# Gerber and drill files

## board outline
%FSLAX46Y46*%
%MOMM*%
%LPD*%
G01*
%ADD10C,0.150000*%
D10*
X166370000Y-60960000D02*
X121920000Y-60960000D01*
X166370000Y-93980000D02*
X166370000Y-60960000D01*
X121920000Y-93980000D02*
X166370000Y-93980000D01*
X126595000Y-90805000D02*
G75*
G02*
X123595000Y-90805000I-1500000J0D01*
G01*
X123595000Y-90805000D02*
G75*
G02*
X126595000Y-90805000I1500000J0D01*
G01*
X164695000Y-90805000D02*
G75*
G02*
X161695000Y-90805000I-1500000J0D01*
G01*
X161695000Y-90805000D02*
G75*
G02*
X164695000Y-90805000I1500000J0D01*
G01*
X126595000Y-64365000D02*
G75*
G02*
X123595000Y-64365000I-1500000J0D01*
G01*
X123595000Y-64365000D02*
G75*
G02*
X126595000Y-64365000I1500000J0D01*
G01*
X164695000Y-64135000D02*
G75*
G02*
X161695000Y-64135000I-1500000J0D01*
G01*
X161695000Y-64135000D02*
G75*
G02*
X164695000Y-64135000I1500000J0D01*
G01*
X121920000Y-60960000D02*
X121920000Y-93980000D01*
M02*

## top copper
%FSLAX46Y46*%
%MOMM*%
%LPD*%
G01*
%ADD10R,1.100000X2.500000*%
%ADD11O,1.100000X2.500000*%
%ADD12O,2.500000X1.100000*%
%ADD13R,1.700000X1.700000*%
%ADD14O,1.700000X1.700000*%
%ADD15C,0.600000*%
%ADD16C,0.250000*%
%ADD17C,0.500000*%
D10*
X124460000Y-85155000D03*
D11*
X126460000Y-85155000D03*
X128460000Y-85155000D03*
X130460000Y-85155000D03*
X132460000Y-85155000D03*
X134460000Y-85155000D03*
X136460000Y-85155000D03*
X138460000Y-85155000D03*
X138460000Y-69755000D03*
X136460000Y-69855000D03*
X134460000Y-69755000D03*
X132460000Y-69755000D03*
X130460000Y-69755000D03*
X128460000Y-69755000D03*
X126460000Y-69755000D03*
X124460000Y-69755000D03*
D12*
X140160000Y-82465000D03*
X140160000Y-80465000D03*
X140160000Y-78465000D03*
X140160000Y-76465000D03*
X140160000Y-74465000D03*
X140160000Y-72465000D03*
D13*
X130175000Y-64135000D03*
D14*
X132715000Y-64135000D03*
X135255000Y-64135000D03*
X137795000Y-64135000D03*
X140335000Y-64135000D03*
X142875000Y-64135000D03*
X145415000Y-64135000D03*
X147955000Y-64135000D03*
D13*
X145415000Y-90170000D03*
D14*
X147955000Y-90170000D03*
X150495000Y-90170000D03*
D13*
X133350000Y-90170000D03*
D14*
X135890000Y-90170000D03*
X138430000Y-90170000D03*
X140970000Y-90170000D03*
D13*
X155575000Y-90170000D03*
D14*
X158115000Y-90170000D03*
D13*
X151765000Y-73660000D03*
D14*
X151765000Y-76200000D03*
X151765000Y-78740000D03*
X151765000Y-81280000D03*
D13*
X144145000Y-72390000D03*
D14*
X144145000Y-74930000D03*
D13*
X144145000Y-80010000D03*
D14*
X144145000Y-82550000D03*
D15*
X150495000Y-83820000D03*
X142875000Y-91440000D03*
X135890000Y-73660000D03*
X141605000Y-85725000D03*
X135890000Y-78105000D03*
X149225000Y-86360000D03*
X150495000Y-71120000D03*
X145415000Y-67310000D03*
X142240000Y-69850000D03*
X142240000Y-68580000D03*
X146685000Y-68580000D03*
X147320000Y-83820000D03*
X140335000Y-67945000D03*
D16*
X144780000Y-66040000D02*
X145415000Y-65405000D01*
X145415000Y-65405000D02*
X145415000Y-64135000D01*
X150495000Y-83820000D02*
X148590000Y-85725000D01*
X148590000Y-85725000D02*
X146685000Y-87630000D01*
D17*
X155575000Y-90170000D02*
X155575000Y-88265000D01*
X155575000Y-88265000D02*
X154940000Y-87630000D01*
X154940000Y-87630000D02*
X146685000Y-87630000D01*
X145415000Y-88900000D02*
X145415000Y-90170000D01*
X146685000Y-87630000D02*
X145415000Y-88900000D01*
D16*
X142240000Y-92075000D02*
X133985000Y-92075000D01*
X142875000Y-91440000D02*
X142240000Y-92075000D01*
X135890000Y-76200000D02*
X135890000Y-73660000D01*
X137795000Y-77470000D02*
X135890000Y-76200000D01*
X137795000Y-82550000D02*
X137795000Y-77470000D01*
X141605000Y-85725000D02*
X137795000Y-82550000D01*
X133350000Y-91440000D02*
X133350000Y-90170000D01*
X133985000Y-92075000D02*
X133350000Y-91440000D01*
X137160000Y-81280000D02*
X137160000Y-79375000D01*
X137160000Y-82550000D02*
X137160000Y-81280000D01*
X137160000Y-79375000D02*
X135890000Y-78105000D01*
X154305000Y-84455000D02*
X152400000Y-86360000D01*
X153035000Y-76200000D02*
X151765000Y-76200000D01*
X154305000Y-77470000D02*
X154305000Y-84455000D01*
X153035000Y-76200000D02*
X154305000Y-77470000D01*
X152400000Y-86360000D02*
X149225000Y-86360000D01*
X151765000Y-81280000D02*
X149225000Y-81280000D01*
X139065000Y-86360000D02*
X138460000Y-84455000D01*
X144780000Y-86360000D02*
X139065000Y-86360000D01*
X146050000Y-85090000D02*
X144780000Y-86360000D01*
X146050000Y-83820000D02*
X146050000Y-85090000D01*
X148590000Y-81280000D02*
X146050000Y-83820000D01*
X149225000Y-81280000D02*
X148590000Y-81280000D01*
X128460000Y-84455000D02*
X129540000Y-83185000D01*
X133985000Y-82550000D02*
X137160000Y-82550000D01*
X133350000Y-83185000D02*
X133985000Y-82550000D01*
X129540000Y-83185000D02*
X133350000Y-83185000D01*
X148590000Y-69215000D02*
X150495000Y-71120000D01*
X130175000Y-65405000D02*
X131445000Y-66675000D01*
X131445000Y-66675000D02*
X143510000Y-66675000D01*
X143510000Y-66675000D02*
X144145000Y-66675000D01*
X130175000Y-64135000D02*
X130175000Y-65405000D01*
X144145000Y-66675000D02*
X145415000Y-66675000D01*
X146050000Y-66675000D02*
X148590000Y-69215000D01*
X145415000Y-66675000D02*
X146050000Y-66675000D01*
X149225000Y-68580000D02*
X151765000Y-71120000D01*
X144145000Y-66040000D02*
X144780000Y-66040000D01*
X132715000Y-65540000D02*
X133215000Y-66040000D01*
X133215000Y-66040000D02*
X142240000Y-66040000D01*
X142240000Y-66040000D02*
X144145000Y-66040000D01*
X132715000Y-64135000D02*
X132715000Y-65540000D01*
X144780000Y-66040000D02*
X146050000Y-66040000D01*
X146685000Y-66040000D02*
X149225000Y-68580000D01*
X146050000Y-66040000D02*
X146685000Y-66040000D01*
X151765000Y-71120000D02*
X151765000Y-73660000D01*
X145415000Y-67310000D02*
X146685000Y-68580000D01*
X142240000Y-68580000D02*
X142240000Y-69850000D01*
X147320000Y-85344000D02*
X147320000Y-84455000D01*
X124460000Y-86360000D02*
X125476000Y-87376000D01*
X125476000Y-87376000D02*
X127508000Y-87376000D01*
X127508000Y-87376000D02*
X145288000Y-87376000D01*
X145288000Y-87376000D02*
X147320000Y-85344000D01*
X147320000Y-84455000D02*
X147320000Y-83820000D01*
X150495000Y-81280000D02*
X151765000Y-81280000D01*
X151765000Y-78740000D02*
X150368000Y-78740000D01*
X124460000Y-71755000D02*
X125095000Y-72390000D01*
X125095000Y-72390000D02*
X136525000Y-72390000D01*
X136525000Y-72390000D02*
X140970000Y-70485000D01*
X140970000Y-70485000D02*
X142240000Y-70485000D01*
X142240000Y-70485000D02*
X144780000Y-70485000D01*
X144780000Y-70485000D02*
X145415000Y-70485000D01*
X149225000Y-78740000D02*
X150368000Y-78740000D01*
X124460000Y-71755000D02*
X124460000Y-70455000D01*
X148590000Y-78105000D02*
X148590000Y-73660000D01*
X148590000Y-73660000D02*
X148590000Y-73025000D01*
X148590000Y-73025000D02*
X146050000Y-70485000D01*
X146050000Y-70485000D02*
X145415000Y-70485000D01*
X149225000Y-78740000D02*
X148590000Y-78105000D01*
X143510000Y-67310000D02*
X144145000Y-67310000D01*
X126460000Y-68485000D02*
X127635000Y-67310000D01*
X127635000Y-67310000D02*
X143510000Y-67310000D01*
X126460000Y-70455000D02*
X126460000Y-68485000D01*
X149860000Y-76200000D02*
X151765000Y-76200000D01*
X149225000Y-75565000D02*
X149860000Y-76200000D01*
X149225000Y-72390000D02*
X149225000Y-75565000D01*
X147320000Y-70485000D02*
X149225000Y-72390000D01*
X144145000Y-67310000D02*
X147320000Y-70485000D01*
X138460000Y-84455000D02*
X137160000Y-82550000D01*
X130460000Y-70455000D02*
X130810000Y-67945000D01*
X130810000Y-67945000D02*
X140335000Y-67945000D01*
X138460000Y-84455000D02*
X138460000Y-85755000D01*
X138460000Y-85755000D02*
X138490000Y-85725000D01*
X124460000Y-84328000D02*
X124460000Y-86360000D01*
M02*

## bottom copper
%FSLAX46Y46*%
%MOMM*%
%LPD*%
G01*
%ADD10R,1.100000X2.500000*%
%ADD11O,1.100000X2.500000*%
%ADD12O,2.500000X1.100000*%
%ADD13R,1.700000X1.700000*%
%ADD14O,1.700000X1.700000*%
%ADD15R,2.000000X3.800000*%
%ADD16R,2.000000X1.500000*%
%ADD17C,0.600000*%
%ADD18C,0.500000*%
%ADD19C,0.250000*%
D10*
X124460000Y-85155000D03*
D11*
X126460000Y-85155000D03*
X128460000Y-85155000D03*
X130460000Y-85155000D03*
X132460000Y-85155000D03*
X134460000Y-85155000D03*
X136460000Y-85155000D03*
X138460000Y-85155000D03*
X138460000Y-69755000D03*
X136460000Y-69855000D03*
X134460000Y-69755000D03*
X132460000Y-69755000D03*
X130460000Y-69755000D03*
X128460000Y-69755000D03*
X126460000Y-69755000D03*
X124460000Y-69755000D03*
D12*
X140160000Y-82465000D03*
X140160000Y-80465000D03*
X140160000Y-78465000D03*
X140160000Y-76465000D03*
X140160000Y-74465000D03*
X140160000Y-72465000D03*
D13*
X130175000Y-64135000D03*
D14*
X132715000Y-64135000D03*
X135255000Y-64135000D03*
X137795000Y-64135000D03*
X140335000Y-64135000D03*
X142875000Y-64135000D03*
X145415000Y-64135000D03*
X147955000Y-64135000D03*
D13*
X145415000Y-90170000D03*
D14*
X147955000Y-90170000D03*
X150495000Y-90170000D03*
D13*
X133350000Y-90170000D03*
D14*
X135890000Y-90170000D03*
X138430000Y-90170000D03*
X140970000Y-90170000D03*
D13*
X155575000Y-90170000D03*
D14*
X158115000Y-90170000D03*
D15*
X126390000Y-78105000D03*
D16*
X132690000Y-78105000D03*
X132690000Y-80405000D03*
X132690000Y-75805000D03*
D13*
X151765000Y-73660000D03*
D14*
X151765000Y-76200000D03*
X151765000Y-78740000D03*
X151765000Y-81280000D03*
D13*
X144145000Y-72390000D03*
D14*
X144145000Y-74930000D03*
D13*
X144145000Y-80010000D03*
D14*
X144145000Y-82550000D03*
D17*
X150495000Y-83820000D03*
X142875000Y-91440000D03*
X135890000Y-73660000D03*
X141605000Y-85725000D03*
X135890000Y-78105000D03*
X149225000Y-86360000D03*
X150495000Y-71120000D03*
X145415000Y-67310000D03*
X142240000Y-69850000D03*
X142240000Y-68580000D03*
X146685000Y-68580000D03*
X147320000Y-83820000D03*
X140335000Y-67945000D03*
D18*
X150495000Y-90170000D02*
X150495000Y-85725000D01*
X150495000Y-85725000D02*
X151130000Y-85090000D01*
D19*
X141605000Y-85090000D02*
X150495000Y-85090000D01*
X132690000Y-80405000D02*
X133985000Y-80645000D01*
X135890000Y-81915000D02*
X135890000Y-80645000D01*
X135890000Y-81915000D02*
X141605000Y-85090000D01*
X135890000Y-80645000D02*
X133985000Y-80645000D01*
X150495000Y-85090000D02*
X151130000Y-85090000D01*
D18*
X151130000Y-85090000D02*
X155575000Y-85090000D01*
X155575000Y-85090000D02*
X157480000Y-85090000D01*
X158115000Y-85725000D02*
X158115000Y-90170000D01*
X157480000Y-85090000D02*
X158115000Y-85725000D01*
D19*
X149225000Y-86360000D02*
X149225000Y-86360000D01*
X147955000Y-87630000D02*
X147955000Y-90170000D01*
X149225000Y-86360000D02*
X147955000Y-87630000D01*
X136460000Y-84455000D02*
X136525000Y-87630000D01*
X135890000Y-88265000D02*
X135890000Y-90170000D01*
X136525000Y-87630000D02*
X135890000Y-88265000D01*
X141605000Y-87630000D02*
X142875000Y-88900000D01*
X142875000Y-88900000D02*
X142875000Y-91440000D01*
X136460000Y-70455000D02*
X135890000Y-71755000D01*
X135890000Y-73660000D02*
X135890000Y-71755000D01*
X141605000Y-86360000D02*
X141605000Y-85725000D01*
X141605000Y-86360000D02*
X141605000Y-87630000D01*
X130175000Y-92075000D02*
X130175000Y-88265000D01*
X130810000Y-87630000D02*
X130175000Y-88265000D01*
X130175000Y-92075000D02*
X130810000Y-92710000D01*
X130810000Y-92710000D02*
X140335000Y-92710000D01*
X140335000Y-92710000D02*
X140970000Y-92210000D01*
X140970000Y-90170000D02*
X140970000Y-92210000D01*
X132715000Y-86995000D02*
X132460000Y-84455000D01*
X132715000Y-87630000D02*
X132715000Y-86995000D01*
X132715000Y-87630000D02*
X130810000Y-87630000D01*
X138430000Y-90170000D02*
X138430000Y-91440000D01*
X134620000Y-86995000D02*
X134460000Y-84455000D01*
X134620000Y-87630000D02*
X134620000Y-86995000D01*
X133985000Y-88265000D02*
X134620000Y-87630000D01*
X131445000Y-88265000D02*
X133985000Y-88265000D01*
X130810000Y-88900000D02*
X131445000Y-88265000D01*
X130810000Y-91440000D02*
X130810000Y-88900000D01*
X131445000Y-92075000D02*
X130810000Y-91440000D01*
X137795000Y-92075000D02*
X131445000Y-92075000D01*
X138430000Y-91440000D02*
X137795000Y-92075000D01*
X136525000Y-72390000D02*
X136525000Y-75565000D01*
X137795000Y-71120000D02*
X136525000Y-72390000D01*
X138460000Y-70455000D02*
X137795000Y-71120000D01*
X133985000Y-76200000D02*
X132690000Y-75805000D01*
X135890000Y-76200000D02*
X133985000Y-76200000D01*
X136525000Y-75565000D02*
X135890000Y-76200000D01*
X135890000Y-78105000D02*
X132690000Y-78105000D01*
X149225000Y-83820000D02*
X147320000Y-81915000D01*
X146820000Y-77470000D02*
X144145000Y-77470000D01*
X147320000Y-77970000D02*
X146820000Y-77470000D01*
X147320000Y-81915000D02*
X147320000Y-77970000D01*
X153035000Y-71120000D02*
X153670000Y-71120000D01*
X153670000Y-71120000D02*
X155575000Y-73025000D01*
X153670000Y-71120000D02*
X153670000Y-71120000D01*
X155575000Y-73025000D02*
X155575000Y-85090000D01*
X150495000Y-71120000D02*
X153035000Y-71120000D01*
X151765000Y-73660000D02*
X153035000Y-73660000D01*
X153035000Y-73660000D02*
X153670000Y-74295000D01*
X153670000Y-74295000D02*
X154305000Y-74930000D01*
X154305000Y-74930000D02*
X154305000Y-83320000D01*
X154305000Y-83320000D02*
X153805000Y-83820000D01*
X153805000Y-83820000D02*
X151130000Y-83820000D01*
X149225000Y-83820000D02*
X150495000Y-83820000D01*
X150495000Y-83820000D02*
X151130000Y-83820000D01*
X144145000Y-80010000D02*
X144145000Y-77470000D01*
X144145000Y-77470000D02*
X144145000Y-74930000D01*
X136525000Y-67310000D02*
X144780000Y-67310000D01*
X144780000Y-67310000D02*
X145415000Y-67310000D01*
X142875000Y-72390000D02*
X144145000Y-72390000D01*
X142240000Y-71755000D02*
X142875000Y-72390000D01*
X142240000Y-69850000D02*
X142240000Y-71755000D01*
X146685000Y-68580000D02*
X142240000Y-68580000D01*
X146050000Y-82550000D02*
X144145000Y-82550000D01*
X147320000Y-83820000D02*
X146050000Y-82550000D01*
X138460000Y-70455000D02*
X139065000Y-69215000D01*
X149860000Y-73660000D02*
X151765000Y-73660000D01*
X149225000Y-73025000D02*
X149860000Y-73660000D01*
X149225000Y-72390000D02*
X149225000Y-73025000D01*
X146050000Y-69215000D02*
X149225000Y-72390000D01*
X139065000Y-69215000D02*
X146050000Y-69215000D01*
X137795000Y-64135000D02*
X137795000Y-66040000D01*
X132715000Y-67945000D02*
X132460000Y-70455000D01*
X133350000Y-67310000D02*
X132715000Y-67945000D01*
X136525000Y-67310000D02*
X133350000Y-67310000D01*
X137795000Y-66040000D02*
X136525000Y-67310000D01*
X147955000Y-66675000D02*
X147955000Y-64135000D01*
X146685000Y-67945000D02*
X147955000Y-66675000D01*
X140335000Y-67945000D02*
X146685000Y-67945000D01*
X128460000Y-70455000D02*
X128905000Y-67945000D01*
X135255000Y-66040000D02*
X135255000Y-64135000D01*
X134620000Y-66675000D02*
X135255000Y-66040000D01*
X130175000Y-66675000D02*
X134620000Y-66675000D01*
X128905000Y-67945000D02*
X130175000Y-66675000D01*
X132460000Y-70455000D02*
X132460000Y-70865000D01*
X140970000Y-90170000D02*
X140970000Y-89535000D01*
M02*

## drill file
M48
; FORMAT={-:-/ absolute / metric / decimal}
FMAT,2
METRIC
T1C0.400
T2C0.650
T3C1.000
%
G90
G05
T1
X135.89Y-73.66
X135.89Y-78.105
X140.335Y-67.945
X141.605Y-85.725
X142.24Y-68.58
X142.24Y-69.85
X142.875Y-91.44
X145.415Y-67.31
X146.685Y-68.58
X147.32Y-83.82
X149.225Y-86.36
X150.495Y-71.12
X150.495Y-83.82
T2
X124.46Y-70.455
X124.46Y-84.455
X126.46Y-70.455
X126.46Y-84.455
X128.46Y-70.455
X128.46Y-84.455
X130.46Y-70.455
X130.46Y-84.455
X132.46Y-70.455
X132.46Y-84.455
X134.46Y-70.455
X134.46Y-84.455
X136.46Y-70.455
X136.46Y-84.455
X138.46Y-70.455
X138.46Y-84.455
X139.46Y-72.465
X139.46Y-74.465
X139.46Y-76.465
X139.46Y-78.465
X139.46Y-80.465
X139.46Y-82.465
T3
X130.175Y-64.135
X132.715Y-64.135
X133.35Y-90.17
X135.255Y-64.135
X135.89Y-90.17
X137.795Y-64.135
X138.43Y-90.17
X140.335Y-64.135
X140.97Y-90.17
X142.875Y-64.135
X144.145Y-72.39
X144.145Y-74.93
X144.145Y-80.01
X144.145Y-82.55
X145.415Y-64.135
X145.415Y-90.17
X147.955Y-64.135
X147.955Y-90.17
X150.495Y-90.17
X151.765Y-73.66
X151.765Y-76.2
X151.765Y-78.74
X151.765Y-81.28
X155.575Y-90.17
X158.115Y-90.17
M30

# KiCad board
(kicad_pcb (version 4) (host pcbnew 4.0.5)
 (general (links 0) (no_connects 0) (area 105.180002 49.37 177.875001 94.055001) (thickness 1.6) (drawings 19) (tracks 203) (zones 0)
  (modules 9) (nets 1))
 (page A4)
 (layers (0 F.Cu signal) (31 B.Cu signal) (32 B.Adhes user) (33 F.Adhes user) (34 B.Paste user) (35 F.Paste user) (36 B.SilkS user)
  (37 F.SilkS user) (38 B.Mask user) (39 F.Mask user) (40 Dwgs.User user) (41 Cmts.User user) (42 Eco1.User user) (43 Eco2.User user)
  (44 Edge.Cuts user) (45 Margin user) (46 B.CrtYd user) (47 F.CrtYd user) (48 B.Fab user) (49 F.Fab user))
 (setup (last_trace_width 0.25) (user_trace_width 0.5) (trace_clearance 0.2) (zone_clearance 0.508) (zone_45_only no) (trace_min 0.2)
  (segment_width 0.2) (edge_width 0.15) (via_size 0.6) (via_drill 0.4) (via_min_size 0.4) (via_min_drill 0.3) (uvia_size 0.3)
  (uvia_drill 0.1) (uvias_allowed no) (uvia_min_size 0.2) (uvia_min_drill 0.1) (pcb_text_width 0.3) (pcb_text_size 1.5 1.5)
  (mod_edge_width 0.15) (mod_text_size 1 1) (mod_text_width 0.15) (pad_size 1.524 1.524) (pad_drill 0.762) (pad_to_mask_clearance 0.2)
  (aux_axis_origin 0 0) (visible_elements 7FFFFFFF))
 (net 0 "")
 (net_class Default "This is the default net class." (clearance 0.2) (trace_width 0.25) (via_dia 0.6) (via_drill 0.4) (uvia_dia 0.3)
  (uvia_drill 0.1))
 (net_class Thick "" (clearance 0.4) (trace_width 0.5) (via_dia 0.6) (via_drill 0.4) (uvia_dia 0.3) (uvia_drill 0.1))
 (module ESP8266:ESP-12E (layer F.Cu) (at 124.46 84.455 90)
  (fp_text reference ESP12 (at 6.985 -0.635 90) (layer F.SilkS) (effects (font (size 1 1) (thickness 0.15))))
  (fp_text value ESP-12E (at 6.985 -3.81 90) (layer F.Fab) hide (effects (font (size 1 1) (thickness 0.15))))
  (pad 1 thru_hole rect (at 0 0 90) (size 2.5 1.1) (drill 0.65 (offset -0.7 0)) (layers *.Cu *.Mask F.SilkS))
  (pad 2 thru_hole oval (at 0 2 90) (size 2.5 1.1) (drill 0.65 (offset -0.7 0)) (layers *.Cu *.Mask F.SilkS))
  (pad 3 thru_hole oval (at 0 4 90) (size 2.5 1.1) (drill 0.65 (offset -0.7 0)) (layers *.Cu *.Mask F.SilkS))
  (pad 4 thru_hole oval (at 0 6 90) (size 2.5 1.1) (drill 0.65 (offset -0.7 0)) (layers *.Cu *.Mask F.SilkS))
  (pad 5 thru_hole oval (at 0 8 90) (size 2.5 1.1) (drill 0.65 (offset -0.7 0)) (layers *.Cu *.Mask F.SilkS))
  (pad 6 thru_hole oval (at 0 10 90) (size 2.5 1.1) (drill 0.65 (offset -0.7 0)) (layers *.Cu *.Mask F.SilkS))
  (pad 7 thru_hole oval (at 0 12 90) (size 2.5 1.1) (drill 0.65 (offset -0.7 0)) (layers *.Cu *.Mask F.SilkS))
  (pad 8 thru_hole oval (at 0 14 90) (size 2.5 1.1) (drill 0.65 (offset -0.7 0)) (layers *.Cu *.Mask F.SilkS))
  (pad 9 thru_hole oval (at 14 14 90) (size 2.5 1.1) (drill 0.65 (offset 0.7 0)) (layers *.Cu *.Mask F.SilkS))
  (pad 10 thru_hole oval (at 14 12 90) (size 2.5 1.1) (drill 0.65 (offset 0.6 0)) (layers *.Cu *.Mask F.SilkS))
  (pad 11 thru_hole oval (at 14 10 90) (size 2.5 1.1) (drill 0.65 (offset 0.7 0)) (layers *.Cu *.Mask F.SilkS))
  (pad 12 thru_hole oval (at 14 8 90) (size 2.5 1.1) (drill 0.65 (offset 0.7 0)) (layers *.Cu *.Mask F.SilkS))
  (pad 13 thru_hole oval (at 14 6 90) (size 2.5 1.1) (drill 0.65 (offset 0.7 0)) (layers *.Cu *.Mask F.SilkS))
  (pad 14 thru_hole oval (at 14 4 90) (size 2.5 1.1) (drill 0.65 (offset 0.7 0)) (layers *.Cu *.Mask F.SilkS))
  (pad 15 thru_hole oval (at 14 2 90) (size 2.5 1.1) (drill 0.65 (offset 0.7 0)) (layers *.Cu *.Mask F.SilkS))
  (pad 16 thru_hole oval (at 14 0 90) (size 2.5 1.1) (drill 0.65 (offset 0.7 0)) (layers *.Cu *.Mask F.SilkS))
  (pad 17 thru_hole oval (at 1.99 15 180) (size 2.5 1.1) (drill 0.65 (offset -0.7 0)) (layers *.Cu *.Mask F.SilkS))
  (pad 18 thru_hole oval (at 3.99 15 180) (size 2.5 1.1) (drill 0.65 (offset -0.7 0)) (layers *.Cu *.Mask F.SilkS))
  (pad 19 thru_hole oval (at 5.99 15 180) (size 2.5 1.1) (drill 0.65 (offset -0.7 0)) (layers *.Cu *.Mask F.SilkS))
  (pad 20 thru_hole oval (at 7.99 15 180) (size 2.5 1.1) (drill 0.65 (offset -0.7 0)) (layers *.Cu *.Mask F.SilkS))
  (pad 21 thru_hole oval (at 9.99 15 180) (size 2.5 1.1) (drill 0.65 (offset -0.7 0)) (layers *.Cu *.Mask F.SilkS))
  (pad 22 thru_hole oval (at 11.99 15 180) (size 2.5 1.1) (drill 0.65 (offset -0.7 0)) (layers *.Cu *.Mask F.SilkS)))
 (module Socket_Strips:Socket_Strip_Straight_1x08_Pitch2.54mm (layer F.Cu) (at 130.175 64.135 90)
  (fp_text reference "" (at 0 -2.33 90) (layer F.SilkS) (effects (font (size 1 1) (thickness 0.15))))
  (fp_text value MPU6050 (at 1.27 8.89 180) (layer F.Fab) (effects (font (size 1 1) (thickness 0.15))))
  (pad 1 thru_hole rect (at 0 0 90) (size 1.7 1.7) (drill 1) (layers *.Cu *.Mask))
  (pad 2 thru_hole oval (at 0 2.54 90) (size 1.7 1.7) (drill 1) (layers *.Cu *.Mask))
  (pad 3 thru_hole oval (at 0 5.08 90) (size 1.7 1.7) (drill 1) (layers *.Cu *.Mask))
  (pad 4 thru_hole oval (at 0 7.62 90) (size 1.7 1.7) (drill 1) (layers *.Cu *.Mask))
  (pad 5 thru_hole oval (at 0 10.16 90) (size 1.7 1.7) (drill 1) (layers *.Cu *.Mask))
  (pad 6 thru_hole oval (at 0 12.7 90) (size 1.7 1.7) (drill 1) (layers *.Cu *.Mask))
  (pad 7 thru_hole oval (at 0 15.24 90) (size 1.7 1.7) (drill 1) (layers *.Cu *.Mask))
  (pad 8 thru_hole oval (at 0 17.78 90) (size 1.7 1.7) (drill 1) (layers *.Cu *.Mask)))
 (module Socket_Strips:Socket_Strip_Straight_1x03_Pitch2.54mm (layer F.Cu) (at 145.415 90.17 90)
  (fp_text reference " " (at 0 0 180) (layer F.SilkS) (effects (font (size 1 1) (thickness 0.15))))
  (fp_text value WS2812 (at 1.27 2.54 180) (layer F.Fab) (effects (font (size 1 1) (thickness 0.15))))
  (pad 1 thru_hole rect (at 0 0 90) (size 1.7 1.7) (drill 1) (layers *.Cu *.Mask))
  (pad 2 thru_hole oval (at 0 2.54 90) (size 1.7 1.7) (drill 1) (layers *.Cu *.Mask))
  (pad 3 thru_hole oval (at 0 5.08 90) (size 1.7 1.7) (drill 1) (layers *.Cu *.Mask)))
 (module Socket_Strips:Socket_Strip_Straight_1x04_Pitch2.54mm (layer F.Cu) (at 133.35 90.17 90)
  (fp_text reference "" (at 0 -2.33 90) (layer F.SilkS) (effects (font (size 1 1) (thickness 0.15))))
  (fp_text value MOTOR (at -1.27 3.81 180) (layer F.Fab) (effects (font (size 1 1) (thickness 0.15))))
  (pad 1 thru_hole rect (at 0 0 90) (size 1.7 1.7) (drill 1) (layers *.Cu *.Mask))
  (pad 2 thru_hole oval (at 0 2.54 90) (size 1.7 1.7) (drill 1) (layers *.Cu *.Mask))
  (pad 3 thru_hole oval (at 0 5.08 90) (size 1.7 1.7) (drill 1) (layers *.Cu *.Mask))
  (pad 4 thru_hole oval (at 0 7.62 90) (size 1.7 1.7) (drill 1) (layers *.Cu *.Mask)))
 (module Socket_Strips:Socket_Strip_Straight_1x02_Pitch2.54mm (layer F.Cu) (at 155.575 90.17 90)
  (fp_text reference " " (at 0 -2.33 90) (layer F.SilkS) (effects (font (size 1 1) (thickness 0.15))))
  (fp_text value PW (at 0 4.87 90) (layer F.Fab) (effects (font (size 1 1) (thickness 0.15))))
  (pad 1 thru_hole rect (at 0 0 90) (size 1.7 1.7) (drill 1) (layers *.Cu *.Mask))
  (pad 2 thru_hole oval (at 0 2.54 90) (size 1.7 1.7) (drill 1) (layers *.Cu *.Mask)))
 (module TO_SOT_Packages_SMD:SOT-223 (layer B.Cu) (at 129.54 78.105 180)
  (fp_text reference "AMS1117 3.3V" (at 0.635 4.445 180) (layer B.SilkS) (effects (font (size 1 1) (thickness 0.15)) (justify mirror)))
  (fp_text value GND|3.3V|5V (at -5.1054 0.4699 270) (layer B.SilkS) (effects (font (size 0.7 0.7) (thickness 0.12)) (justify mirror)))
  (pad 4 smd rect (at 3.15 0 180) (size 2 3.8) (layers B.Cu B.Paste B.Mask))
  (pad 2 smd rect (at -3.15 0 180) (size 2 1.5) (layers B.Cu B.Paste B.Mask))
  (pad 3 smd rect (at -3.15 -2.3 180) (size 2 1.5) (layers B.Cu B.Paste B.Mask))
  (pad 1 smd rect (at -3.15 2.3 180) (size 2 1.5) (layers B.Cu B.Paste B.Mask)))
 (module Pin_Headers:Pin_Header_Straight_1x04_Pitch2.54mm (layer F.Cu) (at 151.765 73.66)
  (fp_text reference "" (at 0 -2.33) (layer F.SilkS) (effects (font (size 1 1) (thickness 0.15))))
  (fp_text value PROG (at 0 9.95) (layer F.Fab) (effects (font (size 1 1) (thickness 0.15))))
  (pad 1 thru_hole rect (at 0 0) (size 1.7 1.7) (drill 1) (layers *.Cu *.Mask))
  (pad 2 thru_hole oval (at 0 2.54) (size 1.7 1.7) (drill 1) (layers *.Cu *.Mask))
  (pad 3 thru_hole oval (at 0 5.08) (size 1.7 1.7) (drill 1) (layers *.Cu *.Mask))
  (pad 4 thru_hole oval (at 0 7.62) (size 1.7 1.7) (drill 1) (layers *.Cu *.Mask)))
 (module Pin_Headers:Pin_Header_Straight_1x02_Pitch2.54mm (layer F.Cu) (at 144.145 72.39)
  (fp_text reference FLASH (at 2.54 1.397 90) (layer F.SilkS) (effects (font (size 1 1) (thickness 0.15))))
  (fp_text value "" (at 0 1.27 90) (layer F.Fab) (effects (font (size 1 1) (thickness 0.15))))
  (pad 1 thru_hole rect (at 0 0) (size 1.7 1.7) (drill 1) (layers *.Cu *.Mask))
  (pad 2 thru_hole oval (at 0 2.54) (size 1.7 1.7) (drill 1) (layers *.Cu *.Mask)))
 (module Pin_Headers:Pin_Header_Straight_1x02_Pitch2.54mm (layer F.Cu) (at 144.145 80.01)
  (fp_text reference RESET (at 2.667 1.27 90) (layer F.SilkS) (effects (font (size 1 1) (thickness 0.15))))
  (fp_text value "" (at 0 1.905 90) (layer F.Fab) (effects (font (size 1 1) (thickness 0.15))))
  (pad 1 thru_hole rect (at 0 0) (size 1.7 1.7) (drill 1) (layers *.Cu *.Mask))
  (pad 2 thru_hole oval (at 0 2.54) (size 1.7 1.7) (drill 1) (layers *.Cu *.Mask)))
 (gr_line (start 166.37 60.96) (end 121.92 60.96) (angle 90) (layer Edge.Cuts) (width 0.15))
 (gr_line (start 166.37 93.98) (end 166.37 60.96) (angle 90) (layer Edge.Cuts) (width 0.15))
 (gr_line (start 121.92 93.98) (end 166.37 93.98) (angle 90) (layer Edge.Cuts) (width 0.15))
 (gr_circle (center 125.095 90.805) (end 125.095 92.305) (layer Edge.Cuts) (width 0.15))
 (gr_circle (center 163.195 90.805) (end 163.195 92.305) (layer Edge.Cuts) (width 0.15))
 (gr_circle (center 125.095 64.365) (end 125.095 62.865) (layer Edge.Cuts) (width 0.15))
 (gr_circle (center 163.195 64.135) (end 163.195 65.635) (layer Edge.Cuts) (width 0.15))
 (gr_line (start 121.92 60.96) (end 121.92 93.98) (angle 90) (layer Edge.Cuts) (width 0.15))
 (segment (start 144.78 66.04) (end 145.415 65.405) (width 0.25) (layer F.Cu) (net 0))
 (segment (start 145.415 65.405) (end 145.415 64.135) (width 0.25) (layer F.Cu) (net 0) (status 800000))
 (segment (start 150.495 83.82) (end 148.59 85.725) (width 0.25) (layer F.Cu) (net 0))
 (segment (start 148.59 85.725) (end 146.685 87.63) (width 0.25) (layer F.Cu) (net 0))
 (via (at 150.495 83.82) (size 0.6) (drill 0.4) (layers F.Cu B.Cu) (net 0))
 (segment (start 155.575 90.17) (end 155.575 88.265) (width 0.5) (layer F.Cu) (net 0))
 (segment (start 155.575 88.265) (end 154.94 87.63) (width 0.5) (layer F.Cu) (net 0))
 (segment (start 154.94 87.63) (end 146.685 87.63) (width 0.5) (layer F.Cu) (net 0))
 (segment (start 150.495 90.17) (end 150.495 85.725) (width 0.5) (layer B.Cu) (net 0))
 (segment (start 150.495 85.725) (end 151.13 85.09) (width 0.5) (layer B.Cu) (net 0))
 (segment (start 141.605 85.09) (end 150.495 85.09) (width 0.25) (layer B.Cu) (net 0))
 (segment (start 132.69 80.405) (end 133.985 80.645) (width 0.25) (layer B.Cu) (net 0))
 (segment (start 135.89 81.915) (end 135.89 80.645) (width 0.25) (layer B.Cu) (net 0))
 (segment (start 135.89 81.915) (end 141.605 85.09) (width 0.25) (layer B.Cu) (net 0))
 (segment (start 135.89 80.645) (end 133.985 80.645) (width 0.25) (layer B.Cu) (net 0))
 (segment (start 150.495 85.09) (end 151.13 85.09) (width 0.25) (layer B.Cu) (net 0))
 (segment (start 151.13 85.09) (end 155.575 85.09) (width 0.5) (layer B.Cu) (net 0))
 (segment (start 155.575 85.09) (end 157.48 85.09) (width 0.5) (layer B.Cu) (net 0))
 (segment (start 158.115 85.725) (end 158.115 90.17) (width 0.5) (layer B.Cu) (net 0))
 (segment (start 157.48 85.09) (end 158.115 85.725) (width 0.5) (layer B.Cu) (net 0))
 (segment (start 149.225 86.36) (end 149.225 86.36) (width 0.25) (layer B.Cu) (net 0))
 (segment (start 147.955 87.63) (end 147.955 90.17) (width 0.25) (layer B.Cu) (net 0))
 (segment (start 149.225 86.36) (end 147.955 87.63) (width 0.25) (layer B.Cu) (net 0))
 (segment (start 145.415 88.9) (end 145.415 90.17) (width 0.5) (layer F.Cu) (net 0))
 (segment (start 146.685 87.63) (end 145.415 88.9) (width 0.5) (layer F.Cu) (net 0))
 (segment (start 136.46 84.455) (end 136.525 87.63) (width 0.25) (layer B.Cu) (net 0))
 (segment (start 135.89 88.265) (end 135.89 90.17) (width 0.25) (layer B.Cu) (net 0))
 (segment (start 136.525 87.63) (end 135.89 88.265) (width 0.25) (layer B.Cu) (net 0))
 (segment (start 142.24 92.075) (end 133.985 92.075) (width 0.25) (layer F.Cu) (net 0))
 (segment (start 141.605 87.63) (end 142.875 88.9) (width 0.25) (layer B.Cu) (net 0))
 (segment (start 142.875 88.9) (end 142.875 91.44) (width 0.25) (layer B.Cu) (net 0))
 (via (at 142.875 91.44) (size 0.6) (drill 0.4) (layers F.Cu B.Cu) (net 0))
 (segment (start 142.875 91.44) (end 142.24 92.075) (width 0.25) (layer F.Cu) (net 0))
 (segment (start 136.46 70.455) (end 135.89 71.755) (width 0.25) (layer B.Cu) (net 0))
 (segment (start 135.89 73.66) (end 135.89 71.755) (width 0.25) (layer B.Cu) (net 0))
 (via (at 135.89 73.66) (size 0.6) (drill 0.4) (layers F.Cu B.Cu) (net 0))
 (segment (start 135.89 76.2) (end 135.89 73.66) (width 0.25) (layer F.Cu) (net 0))
 (segment (start 137.795 77.47) (end 135.89 76.2) (width 0.25) (layer F.Cu) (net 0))
 (segment (start 137.795 82.55) (end 137.795 77.47) (width 0.25) (layer F.Cu) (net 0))
 (segment (start 141.605 85.725) (end 137.795 82.55) (width 0.25) (layer F.Cu) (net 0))
 (via (at 141.605 85.725) (size 0.6) (drill 0.4) (layers F.Cu B.Cu) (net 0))
 (segment (start 141.605 86.36) (end 141.605 85.725) (width 0.25) (layer B.Cu) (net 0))
 (segment (start 141.605 86.36) (end 141.605 87.63) (width 0.25) (layer B.Cu) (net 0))
 (segment (start 133.35 91.44) (end 133.35 90.17) (width 0.25) (layer F.Cu) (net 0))
 (segment (start 133.985 92.075) (end 133.35 91.44) (width 0.25) (layer F.Cu) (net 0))
 (segment (start 130.175 92.075) (end 130.175 88.265) (width 0.25) (layer B.Cu) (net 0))
 (segment (start 130.81 87.63) (end 130.175 88.265) (width 0.25) (layer B.Cu) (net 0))
 (segment (start 130.175 92.075) (end 130.81 92.71) (width 0.25) (layer B.Cu) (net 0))
 (segment (start 130.81 92.71) (end 140.335 92.71) (width 0.25) (layer B.Cu) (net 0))
 (segment (start 140.335 92.71) (end 140.97 92.21) (width 0.25) (layer B.Cu) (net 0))
 (segment (start 140.97 90.17) (end 140.97 92.21) (width 0.25) (layer B.Cu) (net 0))
 (segment (start 132.715 86.995) (end 132.46 84.455) (width 0.25) (layer B.Cu) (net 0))
 (segment (start 132.715 87.63) (end 132.715 86.995) (width 0.25) (layer B.Cu) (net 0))
 (segment (start 132.715 87.63) (end 130.81 87.63) (width 0.25) (layer B.Cu) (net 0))
 (segment (start 138.43 90.17) (end 138.43 91.44) (width 0.25) (layer B.Cu) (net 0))
 (segment (start 134.62 86.995) (end 134.46 84.455) (width 0.25) (layer B.Cu) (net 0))
 (segment (start 134.62 87.63) (end 134.62 86.995) (width 0.25) (layer B.Cu) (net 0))
 (segment (start 133.985 88.265) (end 134.62 87.63) (width 0.25) (layer B.Cu) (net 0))
 (segment (start 131.445 88.265) (end 133.985 88.265) (width 0.25) (layer B.Cu) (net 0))
 (segment (start 130.81 88.9) (end 131.445 88.265) (width 0.25) (layer B.Cu) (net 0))
 (segment (start 130.81 91.44) (end 130.81 88.9) (width 0.25) (layer B.Cu) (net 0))
 (segment (start 131.445 92.075) (end 130.81 91.44) (width 0.25) (layer B.Cu) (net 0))
 (segment (start 137.795 92.075) (end 131.445 92.075) (width 0.25) (layer B.Cu) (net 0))
 (segment (start 138.43 91.44) (end 137.795 92.075) (width 0.25) (layer B.Cu) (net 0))
 (segment (start 136.525 72.39) (end 136.525 75.565) (width 0.25) (layer B.Cu) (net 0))
 (segment (start 137.795 71.12) (end 136.525 72.39) (width 0.25) (layer B.Cu) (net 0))
 (segment (start 138.46 70.455) (end 137.795 71.12) (width 0.25) (layer B.Cu) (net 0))
 (segment (start 133.985 76.2) (end 132.69 75.805) (width 0.25) (layer B.Cu) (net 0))
 (segment (start 135.89 76.2) (end 133.985 76.2) (width 0.25) (layer B.Cu) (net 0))
 (segment (start 136.525 75.565) (end 135.89 76.2) (width 0.25) (layer B.Cu) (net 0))
 (segment (start 137.16 81.28) (end 137.16 79.375) (width 0.25) (layer F.Cu) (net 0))
 (segment (start 137.16 82.55) (end 137.16 81.28) (width 0.25) (layer F.Cu) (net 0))
 (segment (start 135.89 78.105) (end 132.69 78.105) (width 0.25) (layer B.Cu) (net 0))
 (via (at 135.89 78.105) (size 0.6) (drill 0.4) (layers F.Cu B.Cu) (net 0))
 (segment (start 137.16 79.375) (end 135.89 78.105) (width 0.25) (layer F.Cu) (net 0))
 (segment (start 149.225 83.82) (end 147.32 81.915) (width 0.25) (layer B.Cu) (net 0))
 (segment (start 146.82 77.47) (end 144.145 77.47) (width 0.25) (layer B.Cu) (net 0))
 (segment (start 147.32 77.97) (end 146.82 77.47) (width 0.25) (layer B.Cu) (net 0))
 (segment (start 147.32 81.915) (end 147.32 77.97) (width 0.25) (layer B.Cu) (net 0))
 (segment (start 154.305 84.455) (end 152.4 86.36) (width 0.25) (layer F.Cu) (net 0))
 (segment (start 153.035 76.2) (end 151.765 76.2) (width 0.25) (layer F.Cu) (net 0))
 (segment (start 154.305 77.47) (end 154.305 84.455) (width 0.25) (layer F.Cu) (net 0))
 (segment (start 153.035 76.2) (end 154.305 77.47) (width 0.25) (layer F.Cu) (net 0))
 (via (at 149.225 86.36) (size 0.6) (drill 0.4) (layers F.Cu B.Cu) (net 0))
 (segment (start 152.4 86.36) (end 149.225 86.36) (width 0.25) (layer F.Cu) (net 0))
 (segment (start 151.765 81.28) (end 149.225 81.28) (width 0.25) (layer F.Cu) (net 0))
 (segment (start 139.065 86.36) (end 138.46 84.455) (width 0.25) (layer F.Cu) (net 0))
 (segment (start 144.78 86.36) (end 139.065 86.36) (width 0.25) (layer F.Cu) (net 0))
 (segment (start 146.05 85.09) (end 144.78 86.36) (width 0.25) (layer F.Cu) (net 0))
 (segment (start 146.05 83.82) (end 146.05 85.09) (width 0.25) (layer F.Cu) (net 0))
 (segment (start 148.59 81.28) (end 146.05 83.82) (width 0.25) (layer F.Cu) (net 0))
 (segment (start 149.225 81.28) (end 148.59 81.28) (width 0.25) (layer F.Cu) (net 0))
 (segment (start 128.46 84.455) (end 129.54 83.185) (width 0.25) (layer F.Cu) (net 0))
 (segment (start 133.985 82.55) (end 137.16 82.55) (width 0.25) (layer F.Cu) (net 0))
 (segment (start 133.35 83.185) (end 133.985 82.55) (width 0.25) (layer F.Cu) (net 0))
 (segment (start 129.54 83.185) (end 133.35 83.185) (width 0.25) (layer F.Cu) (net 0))
 (segment (start 153.035 71.12) (end 153.67 71.12) (width 0.25) (layer B.Cu) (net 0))
 (segment (start 153.67 71.12) (end 155.575 73.025) (width 0.25) (layer B.Cu) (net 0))
 (segment (start 153.67 71.12) (end 153.67 71.12) (width 0.25) (layer B.Cu) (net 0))
 (segment (start 148.59 69.215) (end 150.495 71.12) (width 0.25) (layer F.Cu) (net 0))
 (segment (start 130.175 65.405) (end 131.445 66.675) (width 0.25) (layer F.Cu) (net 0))
 (segment (start 131.445 66.675) (end 143.51 66.675) (width 0.25) (layer F.Cu) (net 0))
 (segment (start 143.51 66.675) (end 144.145 66.675) (width 0.25) (layer F.Cu) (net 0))
 (segment (start 130.175 64.135) (end 130.175 65.405) (width 0.25) (layer F.Cu) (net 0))
 (segment (start 144.145 66.675) (end 145.415 66.675) (width 0.25) (layer F.Cu) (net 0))
 (segment (start 146.05 66.675) (end 148.59 69.215) (width 0.25) (layer F.Cu) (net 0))
 (segment (start 145.415 66.675) (end 146.05 66.675) (width 0.25) (layer F.Cu) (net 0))
 (segment (start 155.575 73.025) (end 155.575 85.09) (width 0.25) (layer B.Cu) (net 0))
 (segment (start 150.495 71.12) (end 153.035 71.12) (width 0.25) (layer B.Cu) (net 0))
 (via (at 150.495 71.12) (size 0.6) (drill 0.4) (layers F.Cu B.Cu) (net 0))
 (segment (start 149.225 68.58) (end 151.765 71.12) (width 0.25) (layer F.Cu) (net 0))
 (segment (start 144.145 66.04) (end 144.78 66.04) (width 0.25) (layer F.Cu) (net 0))
 (segment (start 132.715 65.54) (end 133.215 66.04) (width 0.25) (layer F.Cu) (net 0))
 (segment (start 133.215 66.04) (end 142.24 66.04) (width 0.25) (layer F.Cu) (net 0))
 (segment (start 142.24 66.04) (end 144.145 66.04) (width 0.25) (layer F.Cu) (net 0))
 (segment (start 132.715 64.135) (end 132.715 65.54) (width 0.25) (layer F.Cu) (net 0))
 (segment (start 144.78 66.04) (end 146.05 66.04) (width 0.25) (layer F.Cu) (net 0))
 (segment (start 146.685 66.04) (end 149.225 68.58) (width 0.25) (layer F.Cu) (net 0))
 (segment (start 146.05 66.04) (end 146.685 66.04) (width 0.25) (layer F.Cu) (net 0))
 (segment (start 151.765 71.12) (end 151.765 73.66) (width 0.25) (layer F.Cu) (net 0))
 (segment (start 151.765 73.66) (end 153.035 73.66) (width 0.25) (layer B.Cu) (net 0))
 (segment (start 153.035 73.66) (end 153.67 74.295) (width 0.25) (layer B.Cu) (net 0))
 (segment (start 153.67 74.295) (end 154.305 74.93) (width 0.25) (layer B.Cu) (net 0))
 (segment (start 154.305 74.93) (end 154.305 83.32) (width 0.25) (layer B.Cu) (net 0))
 (segment (start 154.305 83.32) (end 153.805 83.82) (width 0.25) (layer B.Cu) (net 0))
 (segment (start 153.805 83.82) (end 151.13 83.82) (width 0.25) (layer B.Cu) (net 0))
 (segment (start 149.225 83.82) (end 150.495 83.82) (width 0.25) (layer B.Cu) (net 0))
 (segment (start 150.495 83.82) (end 151.13 83.82) (width 0.25) (layer B.Cu) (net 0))
 (segment (start 144.145 80.01) (end 144.145 77.47) (width 0.25) (layer B.Cu) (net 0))
 (segment (start 144.145 77.47) (end 144.145 74.93) (width 0.25) (layer B.Cu) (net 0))
 (segment (start 145.415 67.31) (end 146.685 68.58) (width 0.25) (layer F.Cu) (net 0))
 (segment (start 136.525 67.31) (end 144.78 67.31) (width 0.25) (layer B.Cu) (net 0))
 (via (at 145.415 67.31) (size 0.6) (drill 0.4) (layers F.Cu B.Cu) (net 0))
 (segment (start 144.78 67.31) (end 145.415 67.31) (width 0.25) (layer B.Cu) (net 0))
 (segment (start 142.875 72.39) (end 144.145 72.39) (width 0.25) (layer B.Cu) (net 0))
 (segment (start 142.24 71.755) (end 142.875 72.39) (width 0.25) (layer B.Cu) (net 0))
 (segment (start 142.24 69.85) (end 142.24 71.755) (width 0.25) (layer B.Cu) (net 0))
 (via (at 142.24 69.85) (size 0.6) (drill 0.4) (layers F.Cu B.Cu) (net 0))
 (segment (start 142.24 68.58) (end 142.24 69.85) (width 0.25) (layer F.Cu) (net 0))
 (via (at 142.24 68.58) (size 0.6) (drill 0.4) (layers F.Cu B.Cu) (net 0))
 (segment (start 146.685 68.58) (end 142.24 68.58) (width 0.25) (layer B.Cu) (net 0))
 (via (at 146.685 68.58) (size 0.6) (drill 0.4) (layers F.Cu B.Cu) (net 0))
 (segment (start 147.32 85.344) (end 147.32 84.455) (width 0.25) (layer F.Cu) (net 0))
 (segment (start 124.46 86.36) (end 125.476 87.376) (width 0.25) (layer F.Cu) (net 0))
 (segment (start 125.476 87.376) (end 127.508 87.376) (width 0.25) (layer F.Cu) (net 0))
 (segment (start 127.508 87.376) (end 145.288 87.376) (width 0.25) (layer F.Cu) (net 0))
 (segment (start 145.288 87.376) (end 147.32 85.344) (width 0.25) (layer F.Cu) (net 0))
 (segment (start 146.05 82.55) (end 144.145 82.55) (width 0.25) (layer B.Cu) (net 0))
 (segment (start 147.32 83.82) (end 146.05 82.55) (width 0.25) (layer B.Cu) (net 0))
 (via (at 147.32 83.82) (size 0.6) (drill 0.4) (layers F.Cu B.Cu) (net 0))
 (segment (start 147.32 84.455) (end 147.32 83.82) (width 0.25) (layer F.Cu) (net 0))
 (segment (start 138.46 70.455) (end 139.065 69.215) (width 0.25) (layer B.Cu) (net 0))
 (segment (start 149.86 73.66) (end 151.765 73.66) (width 0.25) (layer B.Cu) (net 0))
 (segment (start 149.225 73.025) (end 149.86 73.66) (width 0.25) (layer B.Cu) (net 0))
 (segment (start 149.225 72.39) (end 149.225 73.025) (width 0.25) (layer B.Cu) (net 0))
 (segment (start 146.05 69.215) (end 149.225 72.39) (width 0.25) (layer B.Cu) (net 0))
 (segment (start 139.065 69.215) (end 146.05 69.215) (width 0.25) (layer B.Cu) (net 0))
 (segment (start 150.495 81.28) (end 151.765 81.28) (width 0.25) (layer F.Cu) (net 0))
 (segment (start 151.765 78.74) (end 150.368 78.74) (width 0.25) (layer F.Cu) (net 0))
 (segment (start 124.46 71.755) (end 125.095 72.39) (width 0.25) (layer F.Cu) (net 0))
 (segment (start 125.095 72.39) (end 136.525 72.39) (width 0.25) (layer F.Cu) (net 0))
 (segment (start 136.525 72.39) (end 140.97 70.485) (width 0.25) (layer F.Cu) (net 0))
 (segment (start 140.97 70.485) (end 142.24 70.485) (width 0.25) (layer F.Cu) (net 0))
 (segment (start 142.24 70.485) (end 144.78 70.485) (width 0.25) (layer F.Cu) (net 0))
 (segment (start 144.78 70.485) (end 145.415 70.485) (width 0.25) (layer F.Cu) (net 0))
 (segment (start 149.225 78.74) (end 150.368 78.74) (width 0.25) (layer F.Cu) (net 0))
 (segment (start 124.46 71.755) (end 124.46 70.455) (width 0.25) (layer F.Cu) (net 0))
 (segment (start 148.59 78.105) (end 148.59 73.66) (width 0.25) (layer F.Cu) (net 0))
 (segment (start 148.59 73.66) (end 148.59 73.025) (width 0.25) (layer F.Cu) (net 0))
 (segment (start 148.59 73.025) (end 146.05 70.485) (width 0.25) (layer F.Cu) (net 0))
 (segment (start 146.05 70.485) (end 145.415 70.485) (width 0.25) (layer F.Cu) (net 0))
 (segment (start 149.225 78.74) (end 148.59 78.105) (width 0.25) (layer F.Cu) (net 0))
 (segment (start 143.51 67.31) (end 144.145 67.31) (width 0.25) (layer F.Cu) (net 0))
 (segment (start 126.46 68.485) (end 127.635 67.31) (width 0.25) (layer F.Cu) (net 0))
 (segment (start 127.635 67.31) (end 143.51 67.31) (width 0.25) (layer F.Cu) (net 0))
 (segment (start 126.46 70.455) (end 126.46 68.485) (width 0.25) (layer F.Cu) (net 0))
 (segment (start 149.86 76.2) (end 151.765 76.2) (width 0.25) (layer F.Cu) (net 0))
 (segment (start 149.225 75.565) (end 149.86 76.2) (width 0.25) (layer F.Cu) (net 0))
 (segment (start 149.225 72.39) (end 149.225 75.565) (width 0.25) (layer F.Cu) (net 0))
 (segment (start 147.32 70.485) (end 149.225 72.39) (width 0.25) (layer F.Cu) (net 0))
 (segment (start 144.145 67.31) (end 147.32 70.485) (width 0.25) (layer F.Cu) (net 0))
 (segment (start 138.46 84.455) (end 137.16 82.55) (width 0.25) (layer F.Cu) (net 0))
 (segment (start 137.795 64.135) (end 137.795 66.04) (width 0.25) (layer B.Cu) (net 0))
 (segment (start 132.715 67.945) (end 132.46 70.455) (width 0.25) (layer B.Cu) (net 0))
 (segment (start 133.35 67.31) (end 132.715 67.945) (width 0.25) (layer B.Cu) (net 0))
 (segment (start 136.525 67.31) (end 133.35 67.31) (width 0.25) (layer B.Cu) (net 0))
 (segment (start 137.795 66.04) (end 136.525 67.31) (width 0.25) (layer B.Cu) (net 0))
 (segment (start 130.46 70.455) (end 130.81 67.945) (width 0.25) (layer F.Cu) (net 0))
 (segment (start 147.955 66.675) (end 147.955 64.135) (width 0.25) (layer B.Cu) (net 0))
 (segment (start 146.685 67.945) (end 147.955 66.675) (width 0.25) (layer B.Cu) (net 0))
 (segment (start 140.335 67.945) (end 146.685 67.945) (width 0.25) (layer B.Cu) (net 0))
 (via (at 140.335 67.945) (size 0.6) (drill 0.4) (layers F.Cu B.Cu) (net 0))
 (segment (start 130.81 67.945) (end 140.335 67.945) (width 0.25) (layer F.Cu) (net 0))
 (segment (start 128.46 70.455) (end 128.905 67.945) (width 0.25) (layer B.Cu) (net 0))
 (segment (start 135.255 66.04) (end 135.255 64.135) (width 0.25) (layer B.Cu) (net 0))
 (segment (start 134.62 66.675) (end 135.255 66.04) (width 0.25) (layer B.Cu) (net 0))
 (segment (start 130.175 66.675) (end 134.62 66.675) (width 0.25) (layer B.Cu) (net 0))
 (segment (start 128.905 67.945) (end 130.175 66.675) (width 0.25) (layer B.Cu) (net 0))
 (segment (start 132.46 70.455) (end 132.46 70.865) (width 0.25) (layer B.Cu) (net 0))
 (segment (start 138.46 84.455) (end 138.46 85.755) (width 0.25) (layer F.Cu) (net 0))
 (segment (start 138.46 85.755) (end 138.49 85.725) (width 0.25) (layer F.Cu) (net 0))
 (segment (start 124.46 84.328) (end 124.46 86.36) (width 0.25) (layer F.Cu) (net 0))
 (segment (start 140.97 90.17) (end 140.97 89.535) (width 0.25) (layer B.Cu) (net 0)))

